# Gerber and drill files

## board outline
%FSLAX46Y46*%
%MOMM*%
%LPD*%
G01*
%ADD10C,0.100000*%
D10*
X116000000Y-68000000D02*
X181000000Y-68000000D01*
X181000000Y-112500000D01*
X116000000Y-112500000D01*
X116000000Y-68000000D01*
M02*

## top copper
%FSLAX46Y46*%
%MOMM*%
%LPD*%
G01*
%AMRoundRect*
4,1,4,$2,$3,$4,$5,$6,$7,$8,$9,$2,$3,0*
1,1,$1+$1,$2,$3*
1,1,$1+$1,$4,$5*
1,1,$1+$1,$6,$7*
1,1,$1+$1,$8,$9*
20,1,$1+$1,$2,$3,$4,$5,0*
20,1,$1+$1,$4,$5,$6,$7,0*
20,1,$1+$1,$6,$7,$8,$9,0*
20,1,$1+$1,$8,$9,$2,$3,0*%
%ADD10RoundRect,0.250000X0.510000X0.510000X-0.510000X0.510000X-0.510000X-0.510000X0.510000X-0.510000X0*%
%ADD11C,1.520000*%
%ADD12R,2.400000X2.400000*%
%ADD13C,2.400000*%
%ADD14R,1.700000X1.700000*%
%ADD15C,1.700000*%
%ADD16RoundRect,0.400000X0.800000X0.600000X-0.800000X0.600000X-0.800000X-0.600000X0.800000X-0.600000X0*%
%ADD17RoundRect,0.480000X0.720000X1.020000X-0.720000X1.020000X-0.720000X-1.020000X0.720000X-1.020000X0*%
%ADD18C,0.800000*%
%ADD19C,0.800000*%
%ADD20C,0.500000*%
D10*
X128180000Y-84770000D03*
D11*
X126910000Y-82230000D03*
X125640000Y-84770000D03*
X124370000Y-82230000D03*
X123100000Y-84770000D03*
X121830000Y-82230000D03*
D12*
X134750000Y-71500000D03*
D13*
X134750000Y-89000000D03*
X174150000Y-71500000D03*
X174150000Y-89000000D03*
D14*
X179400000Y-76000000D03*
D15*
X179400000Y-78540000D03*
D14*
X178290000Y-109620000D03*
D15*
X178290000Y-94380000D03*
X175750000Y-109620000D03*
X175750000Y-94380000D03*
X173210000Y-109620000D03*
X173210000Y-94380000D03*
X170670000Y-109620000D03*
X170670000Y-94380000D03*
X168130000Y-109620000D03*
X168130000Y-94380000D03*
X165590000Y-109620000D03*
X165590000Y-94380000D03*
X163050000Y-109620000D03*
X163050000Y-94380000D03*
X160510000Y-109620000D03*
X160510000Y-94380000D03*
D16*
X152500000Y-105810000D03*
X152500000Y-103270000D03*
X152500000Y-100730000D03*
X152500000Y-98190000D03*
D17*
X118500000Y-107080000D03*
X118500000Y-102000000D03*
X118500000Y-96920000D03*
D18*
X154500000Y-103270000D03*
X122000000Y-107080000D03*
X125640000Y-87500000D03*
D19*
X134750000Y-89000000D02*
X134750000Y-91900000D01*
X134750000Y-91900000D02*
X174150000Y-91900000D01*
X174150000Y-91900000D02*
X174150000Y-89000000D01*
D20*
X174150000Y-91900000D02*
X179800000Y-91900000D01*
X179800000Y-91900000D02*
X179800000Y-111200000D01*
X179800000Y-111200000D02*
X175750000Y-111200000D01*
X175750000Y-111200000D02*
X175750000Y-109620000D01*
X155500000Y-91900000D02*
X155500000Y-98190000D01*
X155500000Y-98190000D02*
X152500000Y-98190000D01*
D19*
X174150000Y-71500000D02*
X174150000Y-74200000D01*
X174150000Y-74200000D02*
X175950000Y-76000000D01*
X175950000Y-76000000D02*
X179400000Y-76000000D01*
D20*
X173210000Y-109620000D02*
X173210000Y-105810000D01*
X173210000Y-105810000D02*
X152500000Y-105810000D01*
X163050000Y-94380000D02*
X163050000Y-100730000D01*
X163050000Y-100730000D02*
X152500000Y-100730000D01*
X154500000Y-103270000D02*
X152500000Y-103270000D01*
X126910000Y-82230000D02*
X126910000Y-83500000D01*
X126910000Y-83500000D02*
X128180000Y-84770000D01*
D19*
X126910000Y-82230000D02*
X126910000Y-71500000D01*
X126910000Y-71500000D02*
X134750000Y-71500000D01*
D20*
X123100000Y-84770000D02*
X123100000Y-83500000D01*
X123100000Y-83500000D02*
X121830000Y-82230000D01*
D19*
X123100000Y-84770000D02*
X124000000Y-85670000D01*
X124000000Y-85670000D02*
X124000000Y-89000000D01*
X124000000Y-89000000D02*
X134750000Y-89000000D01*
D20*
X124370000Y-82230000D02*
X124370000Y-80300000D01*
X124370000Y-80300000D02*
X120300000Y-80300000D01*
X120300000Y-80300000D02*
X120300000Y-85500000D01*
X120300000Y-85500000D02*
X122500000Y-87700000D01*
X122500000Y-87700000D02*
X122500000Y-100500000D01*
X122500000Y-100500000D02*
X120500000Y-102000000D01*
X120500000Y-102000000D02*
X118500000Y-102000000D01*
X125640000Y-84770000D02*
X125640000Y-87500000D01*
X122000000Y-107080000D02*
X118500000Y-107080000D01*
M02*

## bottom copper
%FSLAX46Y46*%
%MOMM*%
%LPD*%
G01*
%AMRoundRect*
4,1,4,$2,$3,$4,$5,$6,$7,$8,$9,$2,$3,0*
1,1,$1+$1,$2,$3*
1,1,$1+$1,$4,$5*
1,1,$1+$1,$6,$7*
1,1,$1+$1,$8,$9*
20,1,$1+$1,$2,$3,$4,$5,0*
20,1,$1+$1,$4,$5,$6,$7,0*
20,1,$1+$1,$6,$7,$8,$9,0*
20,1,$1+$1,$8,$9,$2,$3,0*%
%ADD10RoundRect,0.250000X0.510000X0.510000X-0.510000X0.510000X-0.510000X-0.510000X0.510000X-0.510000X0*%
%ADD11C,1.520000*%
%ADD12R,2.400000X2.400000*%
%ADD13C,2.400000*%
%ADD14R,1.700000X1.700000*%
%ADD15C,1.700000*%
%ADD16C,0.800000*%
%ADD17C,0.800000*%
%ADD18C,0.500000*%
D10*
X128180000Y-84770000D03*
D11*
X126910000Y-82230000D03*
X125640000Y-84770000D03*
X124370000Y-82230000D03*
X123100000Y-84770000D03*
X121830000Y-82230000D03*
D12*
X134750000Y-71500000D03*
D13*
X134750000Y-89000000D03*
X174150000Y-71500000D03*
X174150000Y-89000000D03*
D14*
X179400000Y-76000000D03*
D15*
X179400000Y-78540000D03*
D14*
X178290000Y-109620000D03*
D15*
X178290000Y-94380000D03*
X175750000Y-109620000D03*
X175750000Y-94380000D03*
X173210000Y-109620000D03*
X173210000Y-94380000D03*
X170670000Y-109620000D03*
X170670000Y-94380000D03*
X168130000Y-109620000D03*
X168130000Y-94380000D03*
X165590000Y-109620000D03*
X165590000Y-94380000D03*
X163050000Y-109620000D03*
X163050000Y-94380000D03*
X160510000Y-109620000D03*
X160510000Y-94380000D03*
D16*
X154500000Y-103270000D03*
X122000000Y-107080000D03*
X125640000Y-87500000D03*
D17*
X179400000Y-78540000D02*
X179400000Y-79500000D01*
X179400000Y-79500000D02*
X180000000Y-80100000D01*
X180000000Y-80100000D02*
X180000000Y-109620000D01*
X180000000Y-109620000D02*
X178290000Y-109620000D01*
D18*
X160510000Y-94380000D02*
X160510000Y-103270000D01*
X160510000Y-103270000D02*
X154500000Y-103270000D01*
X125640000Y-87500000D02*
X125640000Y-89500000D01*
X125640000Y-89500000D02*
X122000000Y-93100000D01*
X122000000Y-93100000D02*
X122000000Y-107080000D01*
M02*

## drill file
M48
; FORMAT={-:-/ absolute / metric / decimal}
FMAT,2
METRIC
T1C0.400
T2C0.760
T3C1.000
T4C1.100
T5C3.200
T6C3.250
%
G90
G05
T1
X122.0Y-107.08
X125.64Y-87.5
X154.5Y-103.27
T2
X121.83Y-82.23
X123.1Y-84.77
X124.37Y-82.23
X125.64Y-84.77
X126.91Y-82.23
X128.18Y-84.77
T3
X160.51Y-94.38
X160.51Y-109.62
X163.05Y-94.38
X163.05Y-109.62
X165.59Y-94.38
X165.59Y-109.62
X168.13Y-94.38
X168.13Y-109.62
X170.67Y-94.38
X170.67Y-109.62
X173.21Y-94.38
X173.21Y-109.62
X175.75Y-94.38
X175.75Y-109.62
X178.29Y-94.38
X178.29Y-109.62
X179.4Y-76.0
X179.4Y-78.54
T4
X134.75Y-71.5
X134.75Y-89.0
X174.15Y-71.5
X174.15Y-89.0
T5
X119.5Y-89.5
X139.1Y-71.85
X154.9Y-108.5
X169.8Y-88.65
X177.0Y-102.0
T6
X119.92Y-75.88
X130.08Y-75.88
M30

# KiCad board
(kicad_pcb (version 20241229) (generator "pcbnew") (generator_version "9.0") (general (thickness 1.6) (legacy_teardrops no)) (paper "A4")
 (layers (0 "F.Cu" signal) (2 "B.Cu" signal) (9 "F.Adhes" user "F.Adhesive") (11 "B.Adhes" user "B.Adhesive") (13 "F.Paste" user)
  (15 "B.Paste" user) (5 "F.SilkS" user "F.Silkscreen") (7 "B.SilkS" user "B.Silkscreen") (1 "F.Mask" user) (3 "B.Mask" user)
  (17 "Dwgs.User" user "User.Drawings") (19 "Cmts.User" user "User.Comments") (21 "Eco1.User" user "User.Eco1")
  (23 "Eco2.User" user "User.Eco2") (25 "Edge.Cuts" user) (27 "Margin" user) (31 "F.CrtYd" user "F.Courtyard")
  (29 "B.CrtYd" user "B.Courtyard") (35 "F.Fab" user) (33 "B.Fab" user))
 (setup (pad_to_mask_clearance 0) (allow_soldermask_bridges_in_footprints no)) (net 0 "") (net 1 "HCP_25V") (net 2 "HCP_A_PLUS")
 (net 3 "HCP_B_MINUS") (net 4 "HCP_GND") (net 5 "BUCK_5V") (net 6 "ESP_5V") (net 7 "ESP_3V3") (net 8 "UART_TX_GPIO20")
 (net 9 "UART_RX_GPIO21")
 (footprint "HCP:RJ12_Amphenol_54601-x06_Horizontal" (layer "F.Cu") (at 128.18 84.77 180)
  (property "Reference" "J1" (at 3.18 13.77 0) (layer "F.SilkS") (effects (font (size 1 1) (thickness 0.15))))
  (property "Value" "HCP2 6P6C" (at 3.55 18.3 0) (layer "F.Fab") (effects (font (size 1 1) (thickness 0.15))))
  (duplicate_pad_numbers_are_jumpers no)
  (pad "" np_thru_hole circle (at -1.9 8.89 180) (size 3.25 3.25) (drill 3.25) (layers "*.Cu" "*.Mask"))
  (pad "" np_thru_hole circle (at 8.26 8.89 180) (size 3.25 3.25) (drill 3.25) (layers "*.Cu" "*.Mask"))
  (pad "1" thru_hole roundrect (at 0 0 180) (size 1.52 1.52) (drill 0.76) (layers "*.Cu" "*.Mask") (remove_unused_layers no)
   (roundrect_rratio 0.1644736842) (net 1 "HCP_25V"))
  (pad "2" thru_hole circle (at 1.27 2.54 180) (size 1.52 1.52) (drill 0.76) (layers "*.Cu" "*.Mask") (remove_unused_layers no)
   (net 1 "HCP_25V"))
  (pad "3" thru_hole circle (at 2.54 0 180) (size 1.52 1.52) (drill 0.76) (layers "*.Cu" "*.Mask") (remove_unused_layers no)
   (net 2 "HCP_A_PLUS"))
  (pad "4" thru_hole circle (at 3.81 2.54 180) (size 1.52 1.52) (drill 0.76) (layers "*.Cu" "*.Mask") (remove_unused_layers no)
   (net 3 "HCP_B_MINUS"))
  (pad "5" thru_hole circle (at 5.08 0 180) (size 1.52 1.52) (drill 0.76) (layers "*.Cu" "*.Mask") (remove_unused_layers no)
   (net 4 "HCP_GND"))
  (pad "6" thru_hole circle (at 6.35 2.54 180) (size 1.52 1.52) (drill 0.76) (layers "*.Cu" "*.Mask") (remove_unused_layers no)
   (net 4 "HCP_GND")))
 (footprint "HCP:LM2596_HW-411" (layer "F.Cu") (at 154.45 80.25 0)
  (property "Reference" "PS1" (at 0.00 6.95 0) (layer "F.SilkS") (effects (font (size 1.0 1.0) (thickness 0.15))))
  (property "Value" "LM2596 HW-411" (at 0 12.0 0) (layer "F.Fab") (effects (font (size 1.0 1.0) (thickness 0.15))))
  (pad "1" thru_hole rect (at -19.7 -8.75) (size 2.4 2.4) (drill 1.1) (layers "*.Cu" "*.Mask") (remove_unused_layers no) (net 1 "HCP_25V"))
  (pad "2" thru_hole circle (at -19.7 8.75) (size 2.4 2.4) (drill 1.1) (layers "*.Cu" "*.Mask") (remove_unused_layers no) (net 4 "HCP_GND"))
  (pad "3" thru_hole circle (at 19.7 -8.75) (size 2.4 2.4) (drill 1.1) (layers "*.Cu" "*.Mask") (remove_unused_layers no) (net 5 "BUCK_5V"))
  (pad "4" thru_hole circle (at 19.7 8.75) (size 2.4 2.4) (drill 1.1) (layers "*.Cu" "*.Mask") (remove_unused_layers no) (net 4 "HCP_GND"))
  (pad "" np_thru_hole circle (at -15.35 -8.4) (size 3.2 3.2) (drill 3.2) (layers "*.Cu" "*.Mask"))
  (pad "" np_thru_hole circle (at 15.35 8.4) (size 3.2 3.2) (drill 3.2) (layers "*.Cu" "*.Mask")))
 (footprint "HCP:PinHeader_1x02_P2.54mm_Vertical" (layer "F.Cu") (at 179.4 76.0 0)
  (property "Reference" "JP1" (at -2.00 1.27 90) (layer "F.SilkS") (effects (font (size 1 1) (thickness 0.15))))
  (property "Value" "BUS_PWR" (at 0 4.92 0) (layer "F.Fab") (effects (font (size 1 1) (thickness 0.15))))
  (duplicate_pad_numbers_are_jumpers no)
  (pad "1" thru_hole rect (at 0 0) (size 1.7 1.7) (drill 1) (layers "*.Cu" "*.Mask") (remove_unused_layers no) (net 5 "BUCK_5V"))
  (pad "2" thru_hole circle (at 0 2.54) (size 1.7 1.7) (drill 1) (layers "*.Cu" "*.Mask") (remove_unused_layers no) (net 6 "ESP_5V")))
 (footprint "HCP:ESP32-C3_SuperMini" (layer "F.Cu") (at 169.4 102.0 270)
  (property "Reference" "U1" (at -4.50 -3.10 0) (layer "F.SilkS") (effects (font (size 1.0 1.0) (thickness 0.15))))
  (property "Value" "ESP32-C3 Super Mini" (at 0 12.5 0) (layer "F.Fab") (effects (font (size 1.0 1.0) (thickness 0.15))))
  (pad "1" thru_hole rect (at 7.62 -8.89 270) (size 1.7 1.7) (drill 1.0) (layers "*.Cu" "*.Mask") (remove_unused_layers no) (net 6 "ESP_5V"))
  (pad "2" thru_hole circle (at -7.62 -8.89 270) (size 1.7 1.7) (drill 1.0) (layers "*.Cu" "*.Mask") (remove_unused_layers no))
  (pad "3" thru_hole circle (at 7.62 -6.35 270) (size 1.7 1.7) (drill 1.0) (layers "*.Cu" "*.Mask") (remove_unused_layers no)
   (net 4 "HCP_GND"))
  (pad "4" thru_hole circle (at -7.62 -6.35 270) (size 1.7 1.7) (drill 1.0) (layers "*.Cu" "*.Mask") (remove_unused_layers no))
  (pad "5" thru_hole circle (at 7.62 -3.81 270) (size 1.7 1.7) (drill 1.0) (layers "*.Cu" "*.Mask") (remove_unused_layers no)
   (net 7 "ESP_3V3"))
  (pad "6" thru_hole circle (at -7.62 -3.81 270) (size 1.7 1.7) (drill 1.0) (layers "*.Cu" "*.Mask") (remove_unused_layers no))
  (pad "7" thru_hole circle (at 7.62 -1.27 270) (size 1.7 1.7) (drill 1.0) (layers "*.Cu" "*.Mask") (remove_unused_layers no))
  (pad "8" thru_hole circle (at -7.62 -1.27 270) (size 1.7 1.7) (drill 1.0) (layers "*.Cu" "*.Mask") (remove_unused_layers no))
  (pad "9" thru_hole circle (at 7.62 1.27 270) (size 1.7 1.7) (drill 1.0) (layers "*.Cu" "*.Mask") (remove_unused_layers no))
  (pad "10" thru_hole circle (at -7.62 1.27 270) (size 1.7 1.7) (drill 1.0) (layers "*.Cu" "*.Mask") (remove_unused_layers no))
  (pad "11" thru_hole circle (at 7.62 3.81 270) (size 1.7 1.7) (drill 1.0) (layers "*.Cu" "*.Mask") (remove_unused_layers no))
  (pad "12" thru_hole circle (at -7.62 3.81 270) (size 1.7 1.7) (drill 1.0) (layers "*.Cu" "*.Mask") (remove_unused_layers no))
  (pad "13" thru_hole circle (at 7.62 6.35 270) (size 1.7 1.7) (drill 1.0) (layers "*.Cu" "*.Mask") (remove_unused_layers no))
  (pad "14" thru_hole circle (at -7.62 6.35 270) (size 1.7 1.7) (drill 1.0) (layers "*.Cu" "*.Mask") (remove_unused_layers no)
   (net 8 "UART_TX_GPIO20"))
  (pad "15" thru_hole circle (at 7.62 8.89 270) (size 1.7 1.7) (drill 1.0) (layers "*.Cu" "*.Mask") (remove_unused_layers no))
  (pad "16" thru_hole circle (at -7.62 8.89 270) (size 1.7 1.7) (drill 1.0) (layers "*.Cu" "*.Mask") (remove_unused_layers no)
   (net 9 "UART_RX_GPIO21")))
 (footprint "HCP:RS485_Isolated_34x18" (layer "F.Cu") (at 135.5 102.0 180)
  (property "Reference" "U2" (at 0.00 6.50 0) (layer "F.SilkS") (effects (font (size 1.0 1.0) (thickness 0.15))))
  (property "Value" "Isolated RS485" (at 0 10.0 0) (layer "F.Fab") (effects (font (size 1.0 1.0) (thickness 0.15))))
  (pad "1" smd roundrect (at -17 -3.81 180) (size 2.4 2.0) (layers "F.Cu" "F.Paste" "F.Mask") (roundrect_rratio 0.2) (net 7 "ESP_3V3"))
  (pad "2" smd roundrect (at -17 -1.27 180) (size 2.4 2.0) (layers "F.Cu" "F.Paste" "F.Mask") (roundrect_rratio 0.2)
   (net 9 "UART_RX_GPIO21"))
  (pad "3" smd roundrect (at -17 1.27 180) (size 2.4 2.0) (layers "F.Cu" "F.Paste" "F.Mask") (roundrect_rratio 0.2) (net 8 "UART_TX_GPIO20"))
  (pad "4" smd roundrect (at -17 3.81 180) (size 2.4 2.0) (layers "F.Cu" "F.Paste" "F.Mask") (roundrect_rratio 0.2) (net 4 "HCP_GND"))
  (pad "5" smd roundrect (at 17 -5.08 180) (size 2.4 3.0) (layers "F.Cu" "F.Paste" "F.Mask") (roundrect_rratio 0.2) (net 2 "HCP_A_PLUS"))
  (pad "6" smd roundrect (at 17 0 180) (size 2.4 3.0) (layers "F.Cu" "F.Paste" "F.Mask") (roundrect_rratio 0.2) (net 3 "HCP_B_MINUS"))
  (pad "7" smd roundrect (at 17 5.08 180) (size 2.4 3.0) (layers "F.Cu" "F.Paste" "F.Mask") (roundrect_rratio 0.2)))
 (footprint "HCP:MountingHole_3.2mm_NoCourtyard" (layer "F.Cu") (at 119.5 89.5 0)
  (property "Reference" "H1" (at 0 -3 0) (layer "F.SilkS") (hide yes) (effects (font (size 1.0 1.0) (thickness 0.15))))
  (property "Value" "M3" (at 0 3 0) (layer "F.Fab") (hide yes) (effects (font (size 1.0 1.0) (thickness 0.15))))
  (pad "" np_thru_hole circle (at 0 0) (size 3.2 3.2) (drill 3.2) (layers "*.Cu" "*.Mask")))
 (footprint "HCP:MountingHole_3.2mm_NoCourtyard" (layer "F.Cu") (at 154.9 108.5 0)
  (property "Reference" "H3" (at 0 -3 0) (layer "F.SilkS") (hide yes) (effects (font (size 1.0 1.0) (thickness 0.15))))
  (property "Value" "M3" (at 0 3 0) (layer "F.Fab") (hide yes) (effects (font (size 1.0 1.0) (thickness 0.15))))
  (pad "" np_thru_hole circle (at 0 0) (size 3.2 3.2) (drill 3.2) (layers "*.Cu" "*.Mask")))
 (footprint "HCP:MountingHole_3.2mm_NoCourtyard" (layer "F.Cu") (at 177.0 102.0 0)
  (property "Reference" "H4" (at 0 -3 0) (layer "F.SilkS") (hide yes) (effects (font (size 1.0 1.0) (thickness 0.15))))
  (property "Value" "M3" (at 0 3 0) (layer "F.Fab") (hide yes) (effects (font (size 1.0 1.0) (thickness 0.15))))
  (pad "" np_thru_hole circle (at 0 0) (size 3.2 3.2) (drill 3.2) (layers "*.Cu" "*.Mask")))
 (segment (start 134.75 89.0) (end 134.75 91.9) (width 0.8) (layer "F.Cu") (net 4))
 (segment (start 134.75 91.9) (end 174.15 91.9) (width 0.8) (layer "F.Cu") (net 4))
 (segment (start 174.15 91.9) (end 174.15 89.0) (width 0.8) (layer "F.Cu") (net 4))
 (segment (start 174.15 91.9) (end 179.8 91.9) (width 0.5) (layer "F.Cu") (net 4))
 (segment (start 179.8 91.9) (end 179.8 111.2) (width 0.5) (layer "F.Cu") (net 4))
 (segment (start 179.8 111.2) (end 175.75 111.2) (width 0.5) (layer "F.Cu") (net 4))
 (segment (start 175.75 111.2) (end 175.75 109.62) (width 0.5) (layer "F.Cu") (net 4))
 (segment (start 155.5 91.9) (end 155.5 98.19) (width 0.5) (layer "F.Cu") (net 4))
 (segment (start 155.5 98.19) (end 152.5 98.19) (width 0.5) (layer "F.Cu") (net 4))
 (segment (start 174.15 71.5) (end 174.15 74.2) (width 0.8) (layer "F.Cu") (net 5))
 (segment (start 174.15 74.2) (end 175.95 76.0) (width 0.8) (layer "F.Cu") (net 5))
 (segment (start 175.95 76.0) (end 179.4 76.0) (width 0.8) (layer "F.Cu") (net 5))
 (segment (start 179.4 78.54) (end 179.4 79.5) (width 0.8) (layer "B.Cu") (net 6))
 (segment (start 179.4 79.5) (end 180.0 80.1) (width 0.8) (layer "B.Cu") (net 6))
 (segment (start 180.0 80.1) (end 180.0 109.62) (width 0.8) (layer "B.Cu") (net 6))
 (segment (start 180.0 109.62) (end 178.29 109.62) (width 0.8) (layer "B.Cu") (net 6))
 (segment (start 173.21 109.62) (end 173.21 105.81) (width 0.5) (layer "F.Cu") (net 7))
 (segment (start 173.21 105.81) (end 152.5 105.81) (width 0.5) (layer "F.Cu") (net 7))
 (segment (start 163.05 94.38) (end 163.05 100.73) (width 0.5) (layer "F.Cu") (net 8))
 (segment (start 163.05 100.73) (end 152.5 100.73) (width 0.5) (layer "F.Cu") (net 8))
 (segment (start 160.51 94.38) (end 160.51 103.27) (width 0.5) (layer "B.Cu") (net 9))
 (segment (start 160.51 103.27) (end 154.5 103.27) (width 0.5) (layer "B.Cu") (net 9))
 (segment (start 154.5 103.27) (end 152.5 103.27) (width 0.5) (layer "F.Cu") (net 9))
 (segment (start 126.91 82.23) (end 126.91 83.5) (width 0.5) (layer "F.Cu") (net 1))
 (segment (start 126.91 83.5) (end 128.18 84.77) (width 0.5) (layer "F.Cu") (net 1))
 (segment (start 126.91 82.23) (end 126.91 71.5) (width 0.8) (layer "F.Cu") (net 1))
 (segment (start 126.91 71.5) (end 134.75 71.5) (width 0.8) (layer "F.Cu") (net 1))
 (segment (start 123.1 84.77) (end 123.1 83.5) (width 0.5) (layer "F.Cu") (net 4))
 (segment (start 123.1 83.5) (end 121.83 82.23) (width 0.5) (layer "F.Cu") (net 4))
 (segment (start 123.1 84.77) (end 124.0 85.67) (width 0.8) (layer "F.Cu") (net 4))
 (segment (start 124.0 85.67) (end 124.0 89.0) (width 0.8) (layer "F.Cu") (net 4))
 (segment (start 124.0 89.0) (end 134.75 89.0) (width 0.8) (layer "F.Cu") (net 4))
 (segment (start 124.37 82.23) (end 124.37 80.3) (width 0.5) (layer "F.Cu") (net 3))
 (segment (start 124.37 80.3) (end 120.3 80.3) (width 0.5) (layer "F.Cu") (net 3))
 (segment (start 120.3 80.3) (end 120.3 85.5) (width 0.5) (layer "F.Cu") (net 3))
 (segment (start 120.3 85.5) (end 122.5 87.7) (width 0.5) (layer "F.Cu") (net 3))
 (segment (start 122.5 87.7) (end 122.5 100.5) (width 0.5) (layer "F.Cu") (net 3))
 (segment (start 122.5 100.5) (end 120.5 102.0) (width 0.5) (layer "F.Cu") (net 3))
 (segment (start 120.5 102.0) (end 118.5 102.0) (width 0.5) (layer "F.Cu") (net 3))
 (segment (start 125.64 84.77) (end 125.64 87.5) (width 0.5) (layer "F.Cu") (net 2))
 (segment (start 125.64 87.5) (end 125.64 89.5) (width 0.5) (layer "B.Cu") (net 2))
 (segment (start 125.64 89.5) (end 122.0 93.1) (width 0.5) (layer "B.Cu") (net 2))
 (segment (start 122.0 93.1) (end 122.0 107.08) (width 0.5) (layer "B.Cu") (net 2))
 (segment (start 122.0 107.08) (end 118.5 107.08) (width 0.5) (layer "F.Cu") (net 2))
 (via (at 154.5 103.27) (size 0.8) (drill 0.4) (layers "F.Cu" "B.Cu") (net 9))
 (via (at 122.0 107.08) (size 0.8) (drill 0.4) (layers "F.Cu" "B.Cu") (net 2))
 (via (at 125.64 87.5) (size 0.8) (drill 0.4) (layers "F.Cu" "B.Cu") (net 2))
 (gr_rect (start 116.0 68.0) (end 181.0 112.5) (stroke (width 0.1) (type default)) (fill none) (layer "Edge.Cuts")))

